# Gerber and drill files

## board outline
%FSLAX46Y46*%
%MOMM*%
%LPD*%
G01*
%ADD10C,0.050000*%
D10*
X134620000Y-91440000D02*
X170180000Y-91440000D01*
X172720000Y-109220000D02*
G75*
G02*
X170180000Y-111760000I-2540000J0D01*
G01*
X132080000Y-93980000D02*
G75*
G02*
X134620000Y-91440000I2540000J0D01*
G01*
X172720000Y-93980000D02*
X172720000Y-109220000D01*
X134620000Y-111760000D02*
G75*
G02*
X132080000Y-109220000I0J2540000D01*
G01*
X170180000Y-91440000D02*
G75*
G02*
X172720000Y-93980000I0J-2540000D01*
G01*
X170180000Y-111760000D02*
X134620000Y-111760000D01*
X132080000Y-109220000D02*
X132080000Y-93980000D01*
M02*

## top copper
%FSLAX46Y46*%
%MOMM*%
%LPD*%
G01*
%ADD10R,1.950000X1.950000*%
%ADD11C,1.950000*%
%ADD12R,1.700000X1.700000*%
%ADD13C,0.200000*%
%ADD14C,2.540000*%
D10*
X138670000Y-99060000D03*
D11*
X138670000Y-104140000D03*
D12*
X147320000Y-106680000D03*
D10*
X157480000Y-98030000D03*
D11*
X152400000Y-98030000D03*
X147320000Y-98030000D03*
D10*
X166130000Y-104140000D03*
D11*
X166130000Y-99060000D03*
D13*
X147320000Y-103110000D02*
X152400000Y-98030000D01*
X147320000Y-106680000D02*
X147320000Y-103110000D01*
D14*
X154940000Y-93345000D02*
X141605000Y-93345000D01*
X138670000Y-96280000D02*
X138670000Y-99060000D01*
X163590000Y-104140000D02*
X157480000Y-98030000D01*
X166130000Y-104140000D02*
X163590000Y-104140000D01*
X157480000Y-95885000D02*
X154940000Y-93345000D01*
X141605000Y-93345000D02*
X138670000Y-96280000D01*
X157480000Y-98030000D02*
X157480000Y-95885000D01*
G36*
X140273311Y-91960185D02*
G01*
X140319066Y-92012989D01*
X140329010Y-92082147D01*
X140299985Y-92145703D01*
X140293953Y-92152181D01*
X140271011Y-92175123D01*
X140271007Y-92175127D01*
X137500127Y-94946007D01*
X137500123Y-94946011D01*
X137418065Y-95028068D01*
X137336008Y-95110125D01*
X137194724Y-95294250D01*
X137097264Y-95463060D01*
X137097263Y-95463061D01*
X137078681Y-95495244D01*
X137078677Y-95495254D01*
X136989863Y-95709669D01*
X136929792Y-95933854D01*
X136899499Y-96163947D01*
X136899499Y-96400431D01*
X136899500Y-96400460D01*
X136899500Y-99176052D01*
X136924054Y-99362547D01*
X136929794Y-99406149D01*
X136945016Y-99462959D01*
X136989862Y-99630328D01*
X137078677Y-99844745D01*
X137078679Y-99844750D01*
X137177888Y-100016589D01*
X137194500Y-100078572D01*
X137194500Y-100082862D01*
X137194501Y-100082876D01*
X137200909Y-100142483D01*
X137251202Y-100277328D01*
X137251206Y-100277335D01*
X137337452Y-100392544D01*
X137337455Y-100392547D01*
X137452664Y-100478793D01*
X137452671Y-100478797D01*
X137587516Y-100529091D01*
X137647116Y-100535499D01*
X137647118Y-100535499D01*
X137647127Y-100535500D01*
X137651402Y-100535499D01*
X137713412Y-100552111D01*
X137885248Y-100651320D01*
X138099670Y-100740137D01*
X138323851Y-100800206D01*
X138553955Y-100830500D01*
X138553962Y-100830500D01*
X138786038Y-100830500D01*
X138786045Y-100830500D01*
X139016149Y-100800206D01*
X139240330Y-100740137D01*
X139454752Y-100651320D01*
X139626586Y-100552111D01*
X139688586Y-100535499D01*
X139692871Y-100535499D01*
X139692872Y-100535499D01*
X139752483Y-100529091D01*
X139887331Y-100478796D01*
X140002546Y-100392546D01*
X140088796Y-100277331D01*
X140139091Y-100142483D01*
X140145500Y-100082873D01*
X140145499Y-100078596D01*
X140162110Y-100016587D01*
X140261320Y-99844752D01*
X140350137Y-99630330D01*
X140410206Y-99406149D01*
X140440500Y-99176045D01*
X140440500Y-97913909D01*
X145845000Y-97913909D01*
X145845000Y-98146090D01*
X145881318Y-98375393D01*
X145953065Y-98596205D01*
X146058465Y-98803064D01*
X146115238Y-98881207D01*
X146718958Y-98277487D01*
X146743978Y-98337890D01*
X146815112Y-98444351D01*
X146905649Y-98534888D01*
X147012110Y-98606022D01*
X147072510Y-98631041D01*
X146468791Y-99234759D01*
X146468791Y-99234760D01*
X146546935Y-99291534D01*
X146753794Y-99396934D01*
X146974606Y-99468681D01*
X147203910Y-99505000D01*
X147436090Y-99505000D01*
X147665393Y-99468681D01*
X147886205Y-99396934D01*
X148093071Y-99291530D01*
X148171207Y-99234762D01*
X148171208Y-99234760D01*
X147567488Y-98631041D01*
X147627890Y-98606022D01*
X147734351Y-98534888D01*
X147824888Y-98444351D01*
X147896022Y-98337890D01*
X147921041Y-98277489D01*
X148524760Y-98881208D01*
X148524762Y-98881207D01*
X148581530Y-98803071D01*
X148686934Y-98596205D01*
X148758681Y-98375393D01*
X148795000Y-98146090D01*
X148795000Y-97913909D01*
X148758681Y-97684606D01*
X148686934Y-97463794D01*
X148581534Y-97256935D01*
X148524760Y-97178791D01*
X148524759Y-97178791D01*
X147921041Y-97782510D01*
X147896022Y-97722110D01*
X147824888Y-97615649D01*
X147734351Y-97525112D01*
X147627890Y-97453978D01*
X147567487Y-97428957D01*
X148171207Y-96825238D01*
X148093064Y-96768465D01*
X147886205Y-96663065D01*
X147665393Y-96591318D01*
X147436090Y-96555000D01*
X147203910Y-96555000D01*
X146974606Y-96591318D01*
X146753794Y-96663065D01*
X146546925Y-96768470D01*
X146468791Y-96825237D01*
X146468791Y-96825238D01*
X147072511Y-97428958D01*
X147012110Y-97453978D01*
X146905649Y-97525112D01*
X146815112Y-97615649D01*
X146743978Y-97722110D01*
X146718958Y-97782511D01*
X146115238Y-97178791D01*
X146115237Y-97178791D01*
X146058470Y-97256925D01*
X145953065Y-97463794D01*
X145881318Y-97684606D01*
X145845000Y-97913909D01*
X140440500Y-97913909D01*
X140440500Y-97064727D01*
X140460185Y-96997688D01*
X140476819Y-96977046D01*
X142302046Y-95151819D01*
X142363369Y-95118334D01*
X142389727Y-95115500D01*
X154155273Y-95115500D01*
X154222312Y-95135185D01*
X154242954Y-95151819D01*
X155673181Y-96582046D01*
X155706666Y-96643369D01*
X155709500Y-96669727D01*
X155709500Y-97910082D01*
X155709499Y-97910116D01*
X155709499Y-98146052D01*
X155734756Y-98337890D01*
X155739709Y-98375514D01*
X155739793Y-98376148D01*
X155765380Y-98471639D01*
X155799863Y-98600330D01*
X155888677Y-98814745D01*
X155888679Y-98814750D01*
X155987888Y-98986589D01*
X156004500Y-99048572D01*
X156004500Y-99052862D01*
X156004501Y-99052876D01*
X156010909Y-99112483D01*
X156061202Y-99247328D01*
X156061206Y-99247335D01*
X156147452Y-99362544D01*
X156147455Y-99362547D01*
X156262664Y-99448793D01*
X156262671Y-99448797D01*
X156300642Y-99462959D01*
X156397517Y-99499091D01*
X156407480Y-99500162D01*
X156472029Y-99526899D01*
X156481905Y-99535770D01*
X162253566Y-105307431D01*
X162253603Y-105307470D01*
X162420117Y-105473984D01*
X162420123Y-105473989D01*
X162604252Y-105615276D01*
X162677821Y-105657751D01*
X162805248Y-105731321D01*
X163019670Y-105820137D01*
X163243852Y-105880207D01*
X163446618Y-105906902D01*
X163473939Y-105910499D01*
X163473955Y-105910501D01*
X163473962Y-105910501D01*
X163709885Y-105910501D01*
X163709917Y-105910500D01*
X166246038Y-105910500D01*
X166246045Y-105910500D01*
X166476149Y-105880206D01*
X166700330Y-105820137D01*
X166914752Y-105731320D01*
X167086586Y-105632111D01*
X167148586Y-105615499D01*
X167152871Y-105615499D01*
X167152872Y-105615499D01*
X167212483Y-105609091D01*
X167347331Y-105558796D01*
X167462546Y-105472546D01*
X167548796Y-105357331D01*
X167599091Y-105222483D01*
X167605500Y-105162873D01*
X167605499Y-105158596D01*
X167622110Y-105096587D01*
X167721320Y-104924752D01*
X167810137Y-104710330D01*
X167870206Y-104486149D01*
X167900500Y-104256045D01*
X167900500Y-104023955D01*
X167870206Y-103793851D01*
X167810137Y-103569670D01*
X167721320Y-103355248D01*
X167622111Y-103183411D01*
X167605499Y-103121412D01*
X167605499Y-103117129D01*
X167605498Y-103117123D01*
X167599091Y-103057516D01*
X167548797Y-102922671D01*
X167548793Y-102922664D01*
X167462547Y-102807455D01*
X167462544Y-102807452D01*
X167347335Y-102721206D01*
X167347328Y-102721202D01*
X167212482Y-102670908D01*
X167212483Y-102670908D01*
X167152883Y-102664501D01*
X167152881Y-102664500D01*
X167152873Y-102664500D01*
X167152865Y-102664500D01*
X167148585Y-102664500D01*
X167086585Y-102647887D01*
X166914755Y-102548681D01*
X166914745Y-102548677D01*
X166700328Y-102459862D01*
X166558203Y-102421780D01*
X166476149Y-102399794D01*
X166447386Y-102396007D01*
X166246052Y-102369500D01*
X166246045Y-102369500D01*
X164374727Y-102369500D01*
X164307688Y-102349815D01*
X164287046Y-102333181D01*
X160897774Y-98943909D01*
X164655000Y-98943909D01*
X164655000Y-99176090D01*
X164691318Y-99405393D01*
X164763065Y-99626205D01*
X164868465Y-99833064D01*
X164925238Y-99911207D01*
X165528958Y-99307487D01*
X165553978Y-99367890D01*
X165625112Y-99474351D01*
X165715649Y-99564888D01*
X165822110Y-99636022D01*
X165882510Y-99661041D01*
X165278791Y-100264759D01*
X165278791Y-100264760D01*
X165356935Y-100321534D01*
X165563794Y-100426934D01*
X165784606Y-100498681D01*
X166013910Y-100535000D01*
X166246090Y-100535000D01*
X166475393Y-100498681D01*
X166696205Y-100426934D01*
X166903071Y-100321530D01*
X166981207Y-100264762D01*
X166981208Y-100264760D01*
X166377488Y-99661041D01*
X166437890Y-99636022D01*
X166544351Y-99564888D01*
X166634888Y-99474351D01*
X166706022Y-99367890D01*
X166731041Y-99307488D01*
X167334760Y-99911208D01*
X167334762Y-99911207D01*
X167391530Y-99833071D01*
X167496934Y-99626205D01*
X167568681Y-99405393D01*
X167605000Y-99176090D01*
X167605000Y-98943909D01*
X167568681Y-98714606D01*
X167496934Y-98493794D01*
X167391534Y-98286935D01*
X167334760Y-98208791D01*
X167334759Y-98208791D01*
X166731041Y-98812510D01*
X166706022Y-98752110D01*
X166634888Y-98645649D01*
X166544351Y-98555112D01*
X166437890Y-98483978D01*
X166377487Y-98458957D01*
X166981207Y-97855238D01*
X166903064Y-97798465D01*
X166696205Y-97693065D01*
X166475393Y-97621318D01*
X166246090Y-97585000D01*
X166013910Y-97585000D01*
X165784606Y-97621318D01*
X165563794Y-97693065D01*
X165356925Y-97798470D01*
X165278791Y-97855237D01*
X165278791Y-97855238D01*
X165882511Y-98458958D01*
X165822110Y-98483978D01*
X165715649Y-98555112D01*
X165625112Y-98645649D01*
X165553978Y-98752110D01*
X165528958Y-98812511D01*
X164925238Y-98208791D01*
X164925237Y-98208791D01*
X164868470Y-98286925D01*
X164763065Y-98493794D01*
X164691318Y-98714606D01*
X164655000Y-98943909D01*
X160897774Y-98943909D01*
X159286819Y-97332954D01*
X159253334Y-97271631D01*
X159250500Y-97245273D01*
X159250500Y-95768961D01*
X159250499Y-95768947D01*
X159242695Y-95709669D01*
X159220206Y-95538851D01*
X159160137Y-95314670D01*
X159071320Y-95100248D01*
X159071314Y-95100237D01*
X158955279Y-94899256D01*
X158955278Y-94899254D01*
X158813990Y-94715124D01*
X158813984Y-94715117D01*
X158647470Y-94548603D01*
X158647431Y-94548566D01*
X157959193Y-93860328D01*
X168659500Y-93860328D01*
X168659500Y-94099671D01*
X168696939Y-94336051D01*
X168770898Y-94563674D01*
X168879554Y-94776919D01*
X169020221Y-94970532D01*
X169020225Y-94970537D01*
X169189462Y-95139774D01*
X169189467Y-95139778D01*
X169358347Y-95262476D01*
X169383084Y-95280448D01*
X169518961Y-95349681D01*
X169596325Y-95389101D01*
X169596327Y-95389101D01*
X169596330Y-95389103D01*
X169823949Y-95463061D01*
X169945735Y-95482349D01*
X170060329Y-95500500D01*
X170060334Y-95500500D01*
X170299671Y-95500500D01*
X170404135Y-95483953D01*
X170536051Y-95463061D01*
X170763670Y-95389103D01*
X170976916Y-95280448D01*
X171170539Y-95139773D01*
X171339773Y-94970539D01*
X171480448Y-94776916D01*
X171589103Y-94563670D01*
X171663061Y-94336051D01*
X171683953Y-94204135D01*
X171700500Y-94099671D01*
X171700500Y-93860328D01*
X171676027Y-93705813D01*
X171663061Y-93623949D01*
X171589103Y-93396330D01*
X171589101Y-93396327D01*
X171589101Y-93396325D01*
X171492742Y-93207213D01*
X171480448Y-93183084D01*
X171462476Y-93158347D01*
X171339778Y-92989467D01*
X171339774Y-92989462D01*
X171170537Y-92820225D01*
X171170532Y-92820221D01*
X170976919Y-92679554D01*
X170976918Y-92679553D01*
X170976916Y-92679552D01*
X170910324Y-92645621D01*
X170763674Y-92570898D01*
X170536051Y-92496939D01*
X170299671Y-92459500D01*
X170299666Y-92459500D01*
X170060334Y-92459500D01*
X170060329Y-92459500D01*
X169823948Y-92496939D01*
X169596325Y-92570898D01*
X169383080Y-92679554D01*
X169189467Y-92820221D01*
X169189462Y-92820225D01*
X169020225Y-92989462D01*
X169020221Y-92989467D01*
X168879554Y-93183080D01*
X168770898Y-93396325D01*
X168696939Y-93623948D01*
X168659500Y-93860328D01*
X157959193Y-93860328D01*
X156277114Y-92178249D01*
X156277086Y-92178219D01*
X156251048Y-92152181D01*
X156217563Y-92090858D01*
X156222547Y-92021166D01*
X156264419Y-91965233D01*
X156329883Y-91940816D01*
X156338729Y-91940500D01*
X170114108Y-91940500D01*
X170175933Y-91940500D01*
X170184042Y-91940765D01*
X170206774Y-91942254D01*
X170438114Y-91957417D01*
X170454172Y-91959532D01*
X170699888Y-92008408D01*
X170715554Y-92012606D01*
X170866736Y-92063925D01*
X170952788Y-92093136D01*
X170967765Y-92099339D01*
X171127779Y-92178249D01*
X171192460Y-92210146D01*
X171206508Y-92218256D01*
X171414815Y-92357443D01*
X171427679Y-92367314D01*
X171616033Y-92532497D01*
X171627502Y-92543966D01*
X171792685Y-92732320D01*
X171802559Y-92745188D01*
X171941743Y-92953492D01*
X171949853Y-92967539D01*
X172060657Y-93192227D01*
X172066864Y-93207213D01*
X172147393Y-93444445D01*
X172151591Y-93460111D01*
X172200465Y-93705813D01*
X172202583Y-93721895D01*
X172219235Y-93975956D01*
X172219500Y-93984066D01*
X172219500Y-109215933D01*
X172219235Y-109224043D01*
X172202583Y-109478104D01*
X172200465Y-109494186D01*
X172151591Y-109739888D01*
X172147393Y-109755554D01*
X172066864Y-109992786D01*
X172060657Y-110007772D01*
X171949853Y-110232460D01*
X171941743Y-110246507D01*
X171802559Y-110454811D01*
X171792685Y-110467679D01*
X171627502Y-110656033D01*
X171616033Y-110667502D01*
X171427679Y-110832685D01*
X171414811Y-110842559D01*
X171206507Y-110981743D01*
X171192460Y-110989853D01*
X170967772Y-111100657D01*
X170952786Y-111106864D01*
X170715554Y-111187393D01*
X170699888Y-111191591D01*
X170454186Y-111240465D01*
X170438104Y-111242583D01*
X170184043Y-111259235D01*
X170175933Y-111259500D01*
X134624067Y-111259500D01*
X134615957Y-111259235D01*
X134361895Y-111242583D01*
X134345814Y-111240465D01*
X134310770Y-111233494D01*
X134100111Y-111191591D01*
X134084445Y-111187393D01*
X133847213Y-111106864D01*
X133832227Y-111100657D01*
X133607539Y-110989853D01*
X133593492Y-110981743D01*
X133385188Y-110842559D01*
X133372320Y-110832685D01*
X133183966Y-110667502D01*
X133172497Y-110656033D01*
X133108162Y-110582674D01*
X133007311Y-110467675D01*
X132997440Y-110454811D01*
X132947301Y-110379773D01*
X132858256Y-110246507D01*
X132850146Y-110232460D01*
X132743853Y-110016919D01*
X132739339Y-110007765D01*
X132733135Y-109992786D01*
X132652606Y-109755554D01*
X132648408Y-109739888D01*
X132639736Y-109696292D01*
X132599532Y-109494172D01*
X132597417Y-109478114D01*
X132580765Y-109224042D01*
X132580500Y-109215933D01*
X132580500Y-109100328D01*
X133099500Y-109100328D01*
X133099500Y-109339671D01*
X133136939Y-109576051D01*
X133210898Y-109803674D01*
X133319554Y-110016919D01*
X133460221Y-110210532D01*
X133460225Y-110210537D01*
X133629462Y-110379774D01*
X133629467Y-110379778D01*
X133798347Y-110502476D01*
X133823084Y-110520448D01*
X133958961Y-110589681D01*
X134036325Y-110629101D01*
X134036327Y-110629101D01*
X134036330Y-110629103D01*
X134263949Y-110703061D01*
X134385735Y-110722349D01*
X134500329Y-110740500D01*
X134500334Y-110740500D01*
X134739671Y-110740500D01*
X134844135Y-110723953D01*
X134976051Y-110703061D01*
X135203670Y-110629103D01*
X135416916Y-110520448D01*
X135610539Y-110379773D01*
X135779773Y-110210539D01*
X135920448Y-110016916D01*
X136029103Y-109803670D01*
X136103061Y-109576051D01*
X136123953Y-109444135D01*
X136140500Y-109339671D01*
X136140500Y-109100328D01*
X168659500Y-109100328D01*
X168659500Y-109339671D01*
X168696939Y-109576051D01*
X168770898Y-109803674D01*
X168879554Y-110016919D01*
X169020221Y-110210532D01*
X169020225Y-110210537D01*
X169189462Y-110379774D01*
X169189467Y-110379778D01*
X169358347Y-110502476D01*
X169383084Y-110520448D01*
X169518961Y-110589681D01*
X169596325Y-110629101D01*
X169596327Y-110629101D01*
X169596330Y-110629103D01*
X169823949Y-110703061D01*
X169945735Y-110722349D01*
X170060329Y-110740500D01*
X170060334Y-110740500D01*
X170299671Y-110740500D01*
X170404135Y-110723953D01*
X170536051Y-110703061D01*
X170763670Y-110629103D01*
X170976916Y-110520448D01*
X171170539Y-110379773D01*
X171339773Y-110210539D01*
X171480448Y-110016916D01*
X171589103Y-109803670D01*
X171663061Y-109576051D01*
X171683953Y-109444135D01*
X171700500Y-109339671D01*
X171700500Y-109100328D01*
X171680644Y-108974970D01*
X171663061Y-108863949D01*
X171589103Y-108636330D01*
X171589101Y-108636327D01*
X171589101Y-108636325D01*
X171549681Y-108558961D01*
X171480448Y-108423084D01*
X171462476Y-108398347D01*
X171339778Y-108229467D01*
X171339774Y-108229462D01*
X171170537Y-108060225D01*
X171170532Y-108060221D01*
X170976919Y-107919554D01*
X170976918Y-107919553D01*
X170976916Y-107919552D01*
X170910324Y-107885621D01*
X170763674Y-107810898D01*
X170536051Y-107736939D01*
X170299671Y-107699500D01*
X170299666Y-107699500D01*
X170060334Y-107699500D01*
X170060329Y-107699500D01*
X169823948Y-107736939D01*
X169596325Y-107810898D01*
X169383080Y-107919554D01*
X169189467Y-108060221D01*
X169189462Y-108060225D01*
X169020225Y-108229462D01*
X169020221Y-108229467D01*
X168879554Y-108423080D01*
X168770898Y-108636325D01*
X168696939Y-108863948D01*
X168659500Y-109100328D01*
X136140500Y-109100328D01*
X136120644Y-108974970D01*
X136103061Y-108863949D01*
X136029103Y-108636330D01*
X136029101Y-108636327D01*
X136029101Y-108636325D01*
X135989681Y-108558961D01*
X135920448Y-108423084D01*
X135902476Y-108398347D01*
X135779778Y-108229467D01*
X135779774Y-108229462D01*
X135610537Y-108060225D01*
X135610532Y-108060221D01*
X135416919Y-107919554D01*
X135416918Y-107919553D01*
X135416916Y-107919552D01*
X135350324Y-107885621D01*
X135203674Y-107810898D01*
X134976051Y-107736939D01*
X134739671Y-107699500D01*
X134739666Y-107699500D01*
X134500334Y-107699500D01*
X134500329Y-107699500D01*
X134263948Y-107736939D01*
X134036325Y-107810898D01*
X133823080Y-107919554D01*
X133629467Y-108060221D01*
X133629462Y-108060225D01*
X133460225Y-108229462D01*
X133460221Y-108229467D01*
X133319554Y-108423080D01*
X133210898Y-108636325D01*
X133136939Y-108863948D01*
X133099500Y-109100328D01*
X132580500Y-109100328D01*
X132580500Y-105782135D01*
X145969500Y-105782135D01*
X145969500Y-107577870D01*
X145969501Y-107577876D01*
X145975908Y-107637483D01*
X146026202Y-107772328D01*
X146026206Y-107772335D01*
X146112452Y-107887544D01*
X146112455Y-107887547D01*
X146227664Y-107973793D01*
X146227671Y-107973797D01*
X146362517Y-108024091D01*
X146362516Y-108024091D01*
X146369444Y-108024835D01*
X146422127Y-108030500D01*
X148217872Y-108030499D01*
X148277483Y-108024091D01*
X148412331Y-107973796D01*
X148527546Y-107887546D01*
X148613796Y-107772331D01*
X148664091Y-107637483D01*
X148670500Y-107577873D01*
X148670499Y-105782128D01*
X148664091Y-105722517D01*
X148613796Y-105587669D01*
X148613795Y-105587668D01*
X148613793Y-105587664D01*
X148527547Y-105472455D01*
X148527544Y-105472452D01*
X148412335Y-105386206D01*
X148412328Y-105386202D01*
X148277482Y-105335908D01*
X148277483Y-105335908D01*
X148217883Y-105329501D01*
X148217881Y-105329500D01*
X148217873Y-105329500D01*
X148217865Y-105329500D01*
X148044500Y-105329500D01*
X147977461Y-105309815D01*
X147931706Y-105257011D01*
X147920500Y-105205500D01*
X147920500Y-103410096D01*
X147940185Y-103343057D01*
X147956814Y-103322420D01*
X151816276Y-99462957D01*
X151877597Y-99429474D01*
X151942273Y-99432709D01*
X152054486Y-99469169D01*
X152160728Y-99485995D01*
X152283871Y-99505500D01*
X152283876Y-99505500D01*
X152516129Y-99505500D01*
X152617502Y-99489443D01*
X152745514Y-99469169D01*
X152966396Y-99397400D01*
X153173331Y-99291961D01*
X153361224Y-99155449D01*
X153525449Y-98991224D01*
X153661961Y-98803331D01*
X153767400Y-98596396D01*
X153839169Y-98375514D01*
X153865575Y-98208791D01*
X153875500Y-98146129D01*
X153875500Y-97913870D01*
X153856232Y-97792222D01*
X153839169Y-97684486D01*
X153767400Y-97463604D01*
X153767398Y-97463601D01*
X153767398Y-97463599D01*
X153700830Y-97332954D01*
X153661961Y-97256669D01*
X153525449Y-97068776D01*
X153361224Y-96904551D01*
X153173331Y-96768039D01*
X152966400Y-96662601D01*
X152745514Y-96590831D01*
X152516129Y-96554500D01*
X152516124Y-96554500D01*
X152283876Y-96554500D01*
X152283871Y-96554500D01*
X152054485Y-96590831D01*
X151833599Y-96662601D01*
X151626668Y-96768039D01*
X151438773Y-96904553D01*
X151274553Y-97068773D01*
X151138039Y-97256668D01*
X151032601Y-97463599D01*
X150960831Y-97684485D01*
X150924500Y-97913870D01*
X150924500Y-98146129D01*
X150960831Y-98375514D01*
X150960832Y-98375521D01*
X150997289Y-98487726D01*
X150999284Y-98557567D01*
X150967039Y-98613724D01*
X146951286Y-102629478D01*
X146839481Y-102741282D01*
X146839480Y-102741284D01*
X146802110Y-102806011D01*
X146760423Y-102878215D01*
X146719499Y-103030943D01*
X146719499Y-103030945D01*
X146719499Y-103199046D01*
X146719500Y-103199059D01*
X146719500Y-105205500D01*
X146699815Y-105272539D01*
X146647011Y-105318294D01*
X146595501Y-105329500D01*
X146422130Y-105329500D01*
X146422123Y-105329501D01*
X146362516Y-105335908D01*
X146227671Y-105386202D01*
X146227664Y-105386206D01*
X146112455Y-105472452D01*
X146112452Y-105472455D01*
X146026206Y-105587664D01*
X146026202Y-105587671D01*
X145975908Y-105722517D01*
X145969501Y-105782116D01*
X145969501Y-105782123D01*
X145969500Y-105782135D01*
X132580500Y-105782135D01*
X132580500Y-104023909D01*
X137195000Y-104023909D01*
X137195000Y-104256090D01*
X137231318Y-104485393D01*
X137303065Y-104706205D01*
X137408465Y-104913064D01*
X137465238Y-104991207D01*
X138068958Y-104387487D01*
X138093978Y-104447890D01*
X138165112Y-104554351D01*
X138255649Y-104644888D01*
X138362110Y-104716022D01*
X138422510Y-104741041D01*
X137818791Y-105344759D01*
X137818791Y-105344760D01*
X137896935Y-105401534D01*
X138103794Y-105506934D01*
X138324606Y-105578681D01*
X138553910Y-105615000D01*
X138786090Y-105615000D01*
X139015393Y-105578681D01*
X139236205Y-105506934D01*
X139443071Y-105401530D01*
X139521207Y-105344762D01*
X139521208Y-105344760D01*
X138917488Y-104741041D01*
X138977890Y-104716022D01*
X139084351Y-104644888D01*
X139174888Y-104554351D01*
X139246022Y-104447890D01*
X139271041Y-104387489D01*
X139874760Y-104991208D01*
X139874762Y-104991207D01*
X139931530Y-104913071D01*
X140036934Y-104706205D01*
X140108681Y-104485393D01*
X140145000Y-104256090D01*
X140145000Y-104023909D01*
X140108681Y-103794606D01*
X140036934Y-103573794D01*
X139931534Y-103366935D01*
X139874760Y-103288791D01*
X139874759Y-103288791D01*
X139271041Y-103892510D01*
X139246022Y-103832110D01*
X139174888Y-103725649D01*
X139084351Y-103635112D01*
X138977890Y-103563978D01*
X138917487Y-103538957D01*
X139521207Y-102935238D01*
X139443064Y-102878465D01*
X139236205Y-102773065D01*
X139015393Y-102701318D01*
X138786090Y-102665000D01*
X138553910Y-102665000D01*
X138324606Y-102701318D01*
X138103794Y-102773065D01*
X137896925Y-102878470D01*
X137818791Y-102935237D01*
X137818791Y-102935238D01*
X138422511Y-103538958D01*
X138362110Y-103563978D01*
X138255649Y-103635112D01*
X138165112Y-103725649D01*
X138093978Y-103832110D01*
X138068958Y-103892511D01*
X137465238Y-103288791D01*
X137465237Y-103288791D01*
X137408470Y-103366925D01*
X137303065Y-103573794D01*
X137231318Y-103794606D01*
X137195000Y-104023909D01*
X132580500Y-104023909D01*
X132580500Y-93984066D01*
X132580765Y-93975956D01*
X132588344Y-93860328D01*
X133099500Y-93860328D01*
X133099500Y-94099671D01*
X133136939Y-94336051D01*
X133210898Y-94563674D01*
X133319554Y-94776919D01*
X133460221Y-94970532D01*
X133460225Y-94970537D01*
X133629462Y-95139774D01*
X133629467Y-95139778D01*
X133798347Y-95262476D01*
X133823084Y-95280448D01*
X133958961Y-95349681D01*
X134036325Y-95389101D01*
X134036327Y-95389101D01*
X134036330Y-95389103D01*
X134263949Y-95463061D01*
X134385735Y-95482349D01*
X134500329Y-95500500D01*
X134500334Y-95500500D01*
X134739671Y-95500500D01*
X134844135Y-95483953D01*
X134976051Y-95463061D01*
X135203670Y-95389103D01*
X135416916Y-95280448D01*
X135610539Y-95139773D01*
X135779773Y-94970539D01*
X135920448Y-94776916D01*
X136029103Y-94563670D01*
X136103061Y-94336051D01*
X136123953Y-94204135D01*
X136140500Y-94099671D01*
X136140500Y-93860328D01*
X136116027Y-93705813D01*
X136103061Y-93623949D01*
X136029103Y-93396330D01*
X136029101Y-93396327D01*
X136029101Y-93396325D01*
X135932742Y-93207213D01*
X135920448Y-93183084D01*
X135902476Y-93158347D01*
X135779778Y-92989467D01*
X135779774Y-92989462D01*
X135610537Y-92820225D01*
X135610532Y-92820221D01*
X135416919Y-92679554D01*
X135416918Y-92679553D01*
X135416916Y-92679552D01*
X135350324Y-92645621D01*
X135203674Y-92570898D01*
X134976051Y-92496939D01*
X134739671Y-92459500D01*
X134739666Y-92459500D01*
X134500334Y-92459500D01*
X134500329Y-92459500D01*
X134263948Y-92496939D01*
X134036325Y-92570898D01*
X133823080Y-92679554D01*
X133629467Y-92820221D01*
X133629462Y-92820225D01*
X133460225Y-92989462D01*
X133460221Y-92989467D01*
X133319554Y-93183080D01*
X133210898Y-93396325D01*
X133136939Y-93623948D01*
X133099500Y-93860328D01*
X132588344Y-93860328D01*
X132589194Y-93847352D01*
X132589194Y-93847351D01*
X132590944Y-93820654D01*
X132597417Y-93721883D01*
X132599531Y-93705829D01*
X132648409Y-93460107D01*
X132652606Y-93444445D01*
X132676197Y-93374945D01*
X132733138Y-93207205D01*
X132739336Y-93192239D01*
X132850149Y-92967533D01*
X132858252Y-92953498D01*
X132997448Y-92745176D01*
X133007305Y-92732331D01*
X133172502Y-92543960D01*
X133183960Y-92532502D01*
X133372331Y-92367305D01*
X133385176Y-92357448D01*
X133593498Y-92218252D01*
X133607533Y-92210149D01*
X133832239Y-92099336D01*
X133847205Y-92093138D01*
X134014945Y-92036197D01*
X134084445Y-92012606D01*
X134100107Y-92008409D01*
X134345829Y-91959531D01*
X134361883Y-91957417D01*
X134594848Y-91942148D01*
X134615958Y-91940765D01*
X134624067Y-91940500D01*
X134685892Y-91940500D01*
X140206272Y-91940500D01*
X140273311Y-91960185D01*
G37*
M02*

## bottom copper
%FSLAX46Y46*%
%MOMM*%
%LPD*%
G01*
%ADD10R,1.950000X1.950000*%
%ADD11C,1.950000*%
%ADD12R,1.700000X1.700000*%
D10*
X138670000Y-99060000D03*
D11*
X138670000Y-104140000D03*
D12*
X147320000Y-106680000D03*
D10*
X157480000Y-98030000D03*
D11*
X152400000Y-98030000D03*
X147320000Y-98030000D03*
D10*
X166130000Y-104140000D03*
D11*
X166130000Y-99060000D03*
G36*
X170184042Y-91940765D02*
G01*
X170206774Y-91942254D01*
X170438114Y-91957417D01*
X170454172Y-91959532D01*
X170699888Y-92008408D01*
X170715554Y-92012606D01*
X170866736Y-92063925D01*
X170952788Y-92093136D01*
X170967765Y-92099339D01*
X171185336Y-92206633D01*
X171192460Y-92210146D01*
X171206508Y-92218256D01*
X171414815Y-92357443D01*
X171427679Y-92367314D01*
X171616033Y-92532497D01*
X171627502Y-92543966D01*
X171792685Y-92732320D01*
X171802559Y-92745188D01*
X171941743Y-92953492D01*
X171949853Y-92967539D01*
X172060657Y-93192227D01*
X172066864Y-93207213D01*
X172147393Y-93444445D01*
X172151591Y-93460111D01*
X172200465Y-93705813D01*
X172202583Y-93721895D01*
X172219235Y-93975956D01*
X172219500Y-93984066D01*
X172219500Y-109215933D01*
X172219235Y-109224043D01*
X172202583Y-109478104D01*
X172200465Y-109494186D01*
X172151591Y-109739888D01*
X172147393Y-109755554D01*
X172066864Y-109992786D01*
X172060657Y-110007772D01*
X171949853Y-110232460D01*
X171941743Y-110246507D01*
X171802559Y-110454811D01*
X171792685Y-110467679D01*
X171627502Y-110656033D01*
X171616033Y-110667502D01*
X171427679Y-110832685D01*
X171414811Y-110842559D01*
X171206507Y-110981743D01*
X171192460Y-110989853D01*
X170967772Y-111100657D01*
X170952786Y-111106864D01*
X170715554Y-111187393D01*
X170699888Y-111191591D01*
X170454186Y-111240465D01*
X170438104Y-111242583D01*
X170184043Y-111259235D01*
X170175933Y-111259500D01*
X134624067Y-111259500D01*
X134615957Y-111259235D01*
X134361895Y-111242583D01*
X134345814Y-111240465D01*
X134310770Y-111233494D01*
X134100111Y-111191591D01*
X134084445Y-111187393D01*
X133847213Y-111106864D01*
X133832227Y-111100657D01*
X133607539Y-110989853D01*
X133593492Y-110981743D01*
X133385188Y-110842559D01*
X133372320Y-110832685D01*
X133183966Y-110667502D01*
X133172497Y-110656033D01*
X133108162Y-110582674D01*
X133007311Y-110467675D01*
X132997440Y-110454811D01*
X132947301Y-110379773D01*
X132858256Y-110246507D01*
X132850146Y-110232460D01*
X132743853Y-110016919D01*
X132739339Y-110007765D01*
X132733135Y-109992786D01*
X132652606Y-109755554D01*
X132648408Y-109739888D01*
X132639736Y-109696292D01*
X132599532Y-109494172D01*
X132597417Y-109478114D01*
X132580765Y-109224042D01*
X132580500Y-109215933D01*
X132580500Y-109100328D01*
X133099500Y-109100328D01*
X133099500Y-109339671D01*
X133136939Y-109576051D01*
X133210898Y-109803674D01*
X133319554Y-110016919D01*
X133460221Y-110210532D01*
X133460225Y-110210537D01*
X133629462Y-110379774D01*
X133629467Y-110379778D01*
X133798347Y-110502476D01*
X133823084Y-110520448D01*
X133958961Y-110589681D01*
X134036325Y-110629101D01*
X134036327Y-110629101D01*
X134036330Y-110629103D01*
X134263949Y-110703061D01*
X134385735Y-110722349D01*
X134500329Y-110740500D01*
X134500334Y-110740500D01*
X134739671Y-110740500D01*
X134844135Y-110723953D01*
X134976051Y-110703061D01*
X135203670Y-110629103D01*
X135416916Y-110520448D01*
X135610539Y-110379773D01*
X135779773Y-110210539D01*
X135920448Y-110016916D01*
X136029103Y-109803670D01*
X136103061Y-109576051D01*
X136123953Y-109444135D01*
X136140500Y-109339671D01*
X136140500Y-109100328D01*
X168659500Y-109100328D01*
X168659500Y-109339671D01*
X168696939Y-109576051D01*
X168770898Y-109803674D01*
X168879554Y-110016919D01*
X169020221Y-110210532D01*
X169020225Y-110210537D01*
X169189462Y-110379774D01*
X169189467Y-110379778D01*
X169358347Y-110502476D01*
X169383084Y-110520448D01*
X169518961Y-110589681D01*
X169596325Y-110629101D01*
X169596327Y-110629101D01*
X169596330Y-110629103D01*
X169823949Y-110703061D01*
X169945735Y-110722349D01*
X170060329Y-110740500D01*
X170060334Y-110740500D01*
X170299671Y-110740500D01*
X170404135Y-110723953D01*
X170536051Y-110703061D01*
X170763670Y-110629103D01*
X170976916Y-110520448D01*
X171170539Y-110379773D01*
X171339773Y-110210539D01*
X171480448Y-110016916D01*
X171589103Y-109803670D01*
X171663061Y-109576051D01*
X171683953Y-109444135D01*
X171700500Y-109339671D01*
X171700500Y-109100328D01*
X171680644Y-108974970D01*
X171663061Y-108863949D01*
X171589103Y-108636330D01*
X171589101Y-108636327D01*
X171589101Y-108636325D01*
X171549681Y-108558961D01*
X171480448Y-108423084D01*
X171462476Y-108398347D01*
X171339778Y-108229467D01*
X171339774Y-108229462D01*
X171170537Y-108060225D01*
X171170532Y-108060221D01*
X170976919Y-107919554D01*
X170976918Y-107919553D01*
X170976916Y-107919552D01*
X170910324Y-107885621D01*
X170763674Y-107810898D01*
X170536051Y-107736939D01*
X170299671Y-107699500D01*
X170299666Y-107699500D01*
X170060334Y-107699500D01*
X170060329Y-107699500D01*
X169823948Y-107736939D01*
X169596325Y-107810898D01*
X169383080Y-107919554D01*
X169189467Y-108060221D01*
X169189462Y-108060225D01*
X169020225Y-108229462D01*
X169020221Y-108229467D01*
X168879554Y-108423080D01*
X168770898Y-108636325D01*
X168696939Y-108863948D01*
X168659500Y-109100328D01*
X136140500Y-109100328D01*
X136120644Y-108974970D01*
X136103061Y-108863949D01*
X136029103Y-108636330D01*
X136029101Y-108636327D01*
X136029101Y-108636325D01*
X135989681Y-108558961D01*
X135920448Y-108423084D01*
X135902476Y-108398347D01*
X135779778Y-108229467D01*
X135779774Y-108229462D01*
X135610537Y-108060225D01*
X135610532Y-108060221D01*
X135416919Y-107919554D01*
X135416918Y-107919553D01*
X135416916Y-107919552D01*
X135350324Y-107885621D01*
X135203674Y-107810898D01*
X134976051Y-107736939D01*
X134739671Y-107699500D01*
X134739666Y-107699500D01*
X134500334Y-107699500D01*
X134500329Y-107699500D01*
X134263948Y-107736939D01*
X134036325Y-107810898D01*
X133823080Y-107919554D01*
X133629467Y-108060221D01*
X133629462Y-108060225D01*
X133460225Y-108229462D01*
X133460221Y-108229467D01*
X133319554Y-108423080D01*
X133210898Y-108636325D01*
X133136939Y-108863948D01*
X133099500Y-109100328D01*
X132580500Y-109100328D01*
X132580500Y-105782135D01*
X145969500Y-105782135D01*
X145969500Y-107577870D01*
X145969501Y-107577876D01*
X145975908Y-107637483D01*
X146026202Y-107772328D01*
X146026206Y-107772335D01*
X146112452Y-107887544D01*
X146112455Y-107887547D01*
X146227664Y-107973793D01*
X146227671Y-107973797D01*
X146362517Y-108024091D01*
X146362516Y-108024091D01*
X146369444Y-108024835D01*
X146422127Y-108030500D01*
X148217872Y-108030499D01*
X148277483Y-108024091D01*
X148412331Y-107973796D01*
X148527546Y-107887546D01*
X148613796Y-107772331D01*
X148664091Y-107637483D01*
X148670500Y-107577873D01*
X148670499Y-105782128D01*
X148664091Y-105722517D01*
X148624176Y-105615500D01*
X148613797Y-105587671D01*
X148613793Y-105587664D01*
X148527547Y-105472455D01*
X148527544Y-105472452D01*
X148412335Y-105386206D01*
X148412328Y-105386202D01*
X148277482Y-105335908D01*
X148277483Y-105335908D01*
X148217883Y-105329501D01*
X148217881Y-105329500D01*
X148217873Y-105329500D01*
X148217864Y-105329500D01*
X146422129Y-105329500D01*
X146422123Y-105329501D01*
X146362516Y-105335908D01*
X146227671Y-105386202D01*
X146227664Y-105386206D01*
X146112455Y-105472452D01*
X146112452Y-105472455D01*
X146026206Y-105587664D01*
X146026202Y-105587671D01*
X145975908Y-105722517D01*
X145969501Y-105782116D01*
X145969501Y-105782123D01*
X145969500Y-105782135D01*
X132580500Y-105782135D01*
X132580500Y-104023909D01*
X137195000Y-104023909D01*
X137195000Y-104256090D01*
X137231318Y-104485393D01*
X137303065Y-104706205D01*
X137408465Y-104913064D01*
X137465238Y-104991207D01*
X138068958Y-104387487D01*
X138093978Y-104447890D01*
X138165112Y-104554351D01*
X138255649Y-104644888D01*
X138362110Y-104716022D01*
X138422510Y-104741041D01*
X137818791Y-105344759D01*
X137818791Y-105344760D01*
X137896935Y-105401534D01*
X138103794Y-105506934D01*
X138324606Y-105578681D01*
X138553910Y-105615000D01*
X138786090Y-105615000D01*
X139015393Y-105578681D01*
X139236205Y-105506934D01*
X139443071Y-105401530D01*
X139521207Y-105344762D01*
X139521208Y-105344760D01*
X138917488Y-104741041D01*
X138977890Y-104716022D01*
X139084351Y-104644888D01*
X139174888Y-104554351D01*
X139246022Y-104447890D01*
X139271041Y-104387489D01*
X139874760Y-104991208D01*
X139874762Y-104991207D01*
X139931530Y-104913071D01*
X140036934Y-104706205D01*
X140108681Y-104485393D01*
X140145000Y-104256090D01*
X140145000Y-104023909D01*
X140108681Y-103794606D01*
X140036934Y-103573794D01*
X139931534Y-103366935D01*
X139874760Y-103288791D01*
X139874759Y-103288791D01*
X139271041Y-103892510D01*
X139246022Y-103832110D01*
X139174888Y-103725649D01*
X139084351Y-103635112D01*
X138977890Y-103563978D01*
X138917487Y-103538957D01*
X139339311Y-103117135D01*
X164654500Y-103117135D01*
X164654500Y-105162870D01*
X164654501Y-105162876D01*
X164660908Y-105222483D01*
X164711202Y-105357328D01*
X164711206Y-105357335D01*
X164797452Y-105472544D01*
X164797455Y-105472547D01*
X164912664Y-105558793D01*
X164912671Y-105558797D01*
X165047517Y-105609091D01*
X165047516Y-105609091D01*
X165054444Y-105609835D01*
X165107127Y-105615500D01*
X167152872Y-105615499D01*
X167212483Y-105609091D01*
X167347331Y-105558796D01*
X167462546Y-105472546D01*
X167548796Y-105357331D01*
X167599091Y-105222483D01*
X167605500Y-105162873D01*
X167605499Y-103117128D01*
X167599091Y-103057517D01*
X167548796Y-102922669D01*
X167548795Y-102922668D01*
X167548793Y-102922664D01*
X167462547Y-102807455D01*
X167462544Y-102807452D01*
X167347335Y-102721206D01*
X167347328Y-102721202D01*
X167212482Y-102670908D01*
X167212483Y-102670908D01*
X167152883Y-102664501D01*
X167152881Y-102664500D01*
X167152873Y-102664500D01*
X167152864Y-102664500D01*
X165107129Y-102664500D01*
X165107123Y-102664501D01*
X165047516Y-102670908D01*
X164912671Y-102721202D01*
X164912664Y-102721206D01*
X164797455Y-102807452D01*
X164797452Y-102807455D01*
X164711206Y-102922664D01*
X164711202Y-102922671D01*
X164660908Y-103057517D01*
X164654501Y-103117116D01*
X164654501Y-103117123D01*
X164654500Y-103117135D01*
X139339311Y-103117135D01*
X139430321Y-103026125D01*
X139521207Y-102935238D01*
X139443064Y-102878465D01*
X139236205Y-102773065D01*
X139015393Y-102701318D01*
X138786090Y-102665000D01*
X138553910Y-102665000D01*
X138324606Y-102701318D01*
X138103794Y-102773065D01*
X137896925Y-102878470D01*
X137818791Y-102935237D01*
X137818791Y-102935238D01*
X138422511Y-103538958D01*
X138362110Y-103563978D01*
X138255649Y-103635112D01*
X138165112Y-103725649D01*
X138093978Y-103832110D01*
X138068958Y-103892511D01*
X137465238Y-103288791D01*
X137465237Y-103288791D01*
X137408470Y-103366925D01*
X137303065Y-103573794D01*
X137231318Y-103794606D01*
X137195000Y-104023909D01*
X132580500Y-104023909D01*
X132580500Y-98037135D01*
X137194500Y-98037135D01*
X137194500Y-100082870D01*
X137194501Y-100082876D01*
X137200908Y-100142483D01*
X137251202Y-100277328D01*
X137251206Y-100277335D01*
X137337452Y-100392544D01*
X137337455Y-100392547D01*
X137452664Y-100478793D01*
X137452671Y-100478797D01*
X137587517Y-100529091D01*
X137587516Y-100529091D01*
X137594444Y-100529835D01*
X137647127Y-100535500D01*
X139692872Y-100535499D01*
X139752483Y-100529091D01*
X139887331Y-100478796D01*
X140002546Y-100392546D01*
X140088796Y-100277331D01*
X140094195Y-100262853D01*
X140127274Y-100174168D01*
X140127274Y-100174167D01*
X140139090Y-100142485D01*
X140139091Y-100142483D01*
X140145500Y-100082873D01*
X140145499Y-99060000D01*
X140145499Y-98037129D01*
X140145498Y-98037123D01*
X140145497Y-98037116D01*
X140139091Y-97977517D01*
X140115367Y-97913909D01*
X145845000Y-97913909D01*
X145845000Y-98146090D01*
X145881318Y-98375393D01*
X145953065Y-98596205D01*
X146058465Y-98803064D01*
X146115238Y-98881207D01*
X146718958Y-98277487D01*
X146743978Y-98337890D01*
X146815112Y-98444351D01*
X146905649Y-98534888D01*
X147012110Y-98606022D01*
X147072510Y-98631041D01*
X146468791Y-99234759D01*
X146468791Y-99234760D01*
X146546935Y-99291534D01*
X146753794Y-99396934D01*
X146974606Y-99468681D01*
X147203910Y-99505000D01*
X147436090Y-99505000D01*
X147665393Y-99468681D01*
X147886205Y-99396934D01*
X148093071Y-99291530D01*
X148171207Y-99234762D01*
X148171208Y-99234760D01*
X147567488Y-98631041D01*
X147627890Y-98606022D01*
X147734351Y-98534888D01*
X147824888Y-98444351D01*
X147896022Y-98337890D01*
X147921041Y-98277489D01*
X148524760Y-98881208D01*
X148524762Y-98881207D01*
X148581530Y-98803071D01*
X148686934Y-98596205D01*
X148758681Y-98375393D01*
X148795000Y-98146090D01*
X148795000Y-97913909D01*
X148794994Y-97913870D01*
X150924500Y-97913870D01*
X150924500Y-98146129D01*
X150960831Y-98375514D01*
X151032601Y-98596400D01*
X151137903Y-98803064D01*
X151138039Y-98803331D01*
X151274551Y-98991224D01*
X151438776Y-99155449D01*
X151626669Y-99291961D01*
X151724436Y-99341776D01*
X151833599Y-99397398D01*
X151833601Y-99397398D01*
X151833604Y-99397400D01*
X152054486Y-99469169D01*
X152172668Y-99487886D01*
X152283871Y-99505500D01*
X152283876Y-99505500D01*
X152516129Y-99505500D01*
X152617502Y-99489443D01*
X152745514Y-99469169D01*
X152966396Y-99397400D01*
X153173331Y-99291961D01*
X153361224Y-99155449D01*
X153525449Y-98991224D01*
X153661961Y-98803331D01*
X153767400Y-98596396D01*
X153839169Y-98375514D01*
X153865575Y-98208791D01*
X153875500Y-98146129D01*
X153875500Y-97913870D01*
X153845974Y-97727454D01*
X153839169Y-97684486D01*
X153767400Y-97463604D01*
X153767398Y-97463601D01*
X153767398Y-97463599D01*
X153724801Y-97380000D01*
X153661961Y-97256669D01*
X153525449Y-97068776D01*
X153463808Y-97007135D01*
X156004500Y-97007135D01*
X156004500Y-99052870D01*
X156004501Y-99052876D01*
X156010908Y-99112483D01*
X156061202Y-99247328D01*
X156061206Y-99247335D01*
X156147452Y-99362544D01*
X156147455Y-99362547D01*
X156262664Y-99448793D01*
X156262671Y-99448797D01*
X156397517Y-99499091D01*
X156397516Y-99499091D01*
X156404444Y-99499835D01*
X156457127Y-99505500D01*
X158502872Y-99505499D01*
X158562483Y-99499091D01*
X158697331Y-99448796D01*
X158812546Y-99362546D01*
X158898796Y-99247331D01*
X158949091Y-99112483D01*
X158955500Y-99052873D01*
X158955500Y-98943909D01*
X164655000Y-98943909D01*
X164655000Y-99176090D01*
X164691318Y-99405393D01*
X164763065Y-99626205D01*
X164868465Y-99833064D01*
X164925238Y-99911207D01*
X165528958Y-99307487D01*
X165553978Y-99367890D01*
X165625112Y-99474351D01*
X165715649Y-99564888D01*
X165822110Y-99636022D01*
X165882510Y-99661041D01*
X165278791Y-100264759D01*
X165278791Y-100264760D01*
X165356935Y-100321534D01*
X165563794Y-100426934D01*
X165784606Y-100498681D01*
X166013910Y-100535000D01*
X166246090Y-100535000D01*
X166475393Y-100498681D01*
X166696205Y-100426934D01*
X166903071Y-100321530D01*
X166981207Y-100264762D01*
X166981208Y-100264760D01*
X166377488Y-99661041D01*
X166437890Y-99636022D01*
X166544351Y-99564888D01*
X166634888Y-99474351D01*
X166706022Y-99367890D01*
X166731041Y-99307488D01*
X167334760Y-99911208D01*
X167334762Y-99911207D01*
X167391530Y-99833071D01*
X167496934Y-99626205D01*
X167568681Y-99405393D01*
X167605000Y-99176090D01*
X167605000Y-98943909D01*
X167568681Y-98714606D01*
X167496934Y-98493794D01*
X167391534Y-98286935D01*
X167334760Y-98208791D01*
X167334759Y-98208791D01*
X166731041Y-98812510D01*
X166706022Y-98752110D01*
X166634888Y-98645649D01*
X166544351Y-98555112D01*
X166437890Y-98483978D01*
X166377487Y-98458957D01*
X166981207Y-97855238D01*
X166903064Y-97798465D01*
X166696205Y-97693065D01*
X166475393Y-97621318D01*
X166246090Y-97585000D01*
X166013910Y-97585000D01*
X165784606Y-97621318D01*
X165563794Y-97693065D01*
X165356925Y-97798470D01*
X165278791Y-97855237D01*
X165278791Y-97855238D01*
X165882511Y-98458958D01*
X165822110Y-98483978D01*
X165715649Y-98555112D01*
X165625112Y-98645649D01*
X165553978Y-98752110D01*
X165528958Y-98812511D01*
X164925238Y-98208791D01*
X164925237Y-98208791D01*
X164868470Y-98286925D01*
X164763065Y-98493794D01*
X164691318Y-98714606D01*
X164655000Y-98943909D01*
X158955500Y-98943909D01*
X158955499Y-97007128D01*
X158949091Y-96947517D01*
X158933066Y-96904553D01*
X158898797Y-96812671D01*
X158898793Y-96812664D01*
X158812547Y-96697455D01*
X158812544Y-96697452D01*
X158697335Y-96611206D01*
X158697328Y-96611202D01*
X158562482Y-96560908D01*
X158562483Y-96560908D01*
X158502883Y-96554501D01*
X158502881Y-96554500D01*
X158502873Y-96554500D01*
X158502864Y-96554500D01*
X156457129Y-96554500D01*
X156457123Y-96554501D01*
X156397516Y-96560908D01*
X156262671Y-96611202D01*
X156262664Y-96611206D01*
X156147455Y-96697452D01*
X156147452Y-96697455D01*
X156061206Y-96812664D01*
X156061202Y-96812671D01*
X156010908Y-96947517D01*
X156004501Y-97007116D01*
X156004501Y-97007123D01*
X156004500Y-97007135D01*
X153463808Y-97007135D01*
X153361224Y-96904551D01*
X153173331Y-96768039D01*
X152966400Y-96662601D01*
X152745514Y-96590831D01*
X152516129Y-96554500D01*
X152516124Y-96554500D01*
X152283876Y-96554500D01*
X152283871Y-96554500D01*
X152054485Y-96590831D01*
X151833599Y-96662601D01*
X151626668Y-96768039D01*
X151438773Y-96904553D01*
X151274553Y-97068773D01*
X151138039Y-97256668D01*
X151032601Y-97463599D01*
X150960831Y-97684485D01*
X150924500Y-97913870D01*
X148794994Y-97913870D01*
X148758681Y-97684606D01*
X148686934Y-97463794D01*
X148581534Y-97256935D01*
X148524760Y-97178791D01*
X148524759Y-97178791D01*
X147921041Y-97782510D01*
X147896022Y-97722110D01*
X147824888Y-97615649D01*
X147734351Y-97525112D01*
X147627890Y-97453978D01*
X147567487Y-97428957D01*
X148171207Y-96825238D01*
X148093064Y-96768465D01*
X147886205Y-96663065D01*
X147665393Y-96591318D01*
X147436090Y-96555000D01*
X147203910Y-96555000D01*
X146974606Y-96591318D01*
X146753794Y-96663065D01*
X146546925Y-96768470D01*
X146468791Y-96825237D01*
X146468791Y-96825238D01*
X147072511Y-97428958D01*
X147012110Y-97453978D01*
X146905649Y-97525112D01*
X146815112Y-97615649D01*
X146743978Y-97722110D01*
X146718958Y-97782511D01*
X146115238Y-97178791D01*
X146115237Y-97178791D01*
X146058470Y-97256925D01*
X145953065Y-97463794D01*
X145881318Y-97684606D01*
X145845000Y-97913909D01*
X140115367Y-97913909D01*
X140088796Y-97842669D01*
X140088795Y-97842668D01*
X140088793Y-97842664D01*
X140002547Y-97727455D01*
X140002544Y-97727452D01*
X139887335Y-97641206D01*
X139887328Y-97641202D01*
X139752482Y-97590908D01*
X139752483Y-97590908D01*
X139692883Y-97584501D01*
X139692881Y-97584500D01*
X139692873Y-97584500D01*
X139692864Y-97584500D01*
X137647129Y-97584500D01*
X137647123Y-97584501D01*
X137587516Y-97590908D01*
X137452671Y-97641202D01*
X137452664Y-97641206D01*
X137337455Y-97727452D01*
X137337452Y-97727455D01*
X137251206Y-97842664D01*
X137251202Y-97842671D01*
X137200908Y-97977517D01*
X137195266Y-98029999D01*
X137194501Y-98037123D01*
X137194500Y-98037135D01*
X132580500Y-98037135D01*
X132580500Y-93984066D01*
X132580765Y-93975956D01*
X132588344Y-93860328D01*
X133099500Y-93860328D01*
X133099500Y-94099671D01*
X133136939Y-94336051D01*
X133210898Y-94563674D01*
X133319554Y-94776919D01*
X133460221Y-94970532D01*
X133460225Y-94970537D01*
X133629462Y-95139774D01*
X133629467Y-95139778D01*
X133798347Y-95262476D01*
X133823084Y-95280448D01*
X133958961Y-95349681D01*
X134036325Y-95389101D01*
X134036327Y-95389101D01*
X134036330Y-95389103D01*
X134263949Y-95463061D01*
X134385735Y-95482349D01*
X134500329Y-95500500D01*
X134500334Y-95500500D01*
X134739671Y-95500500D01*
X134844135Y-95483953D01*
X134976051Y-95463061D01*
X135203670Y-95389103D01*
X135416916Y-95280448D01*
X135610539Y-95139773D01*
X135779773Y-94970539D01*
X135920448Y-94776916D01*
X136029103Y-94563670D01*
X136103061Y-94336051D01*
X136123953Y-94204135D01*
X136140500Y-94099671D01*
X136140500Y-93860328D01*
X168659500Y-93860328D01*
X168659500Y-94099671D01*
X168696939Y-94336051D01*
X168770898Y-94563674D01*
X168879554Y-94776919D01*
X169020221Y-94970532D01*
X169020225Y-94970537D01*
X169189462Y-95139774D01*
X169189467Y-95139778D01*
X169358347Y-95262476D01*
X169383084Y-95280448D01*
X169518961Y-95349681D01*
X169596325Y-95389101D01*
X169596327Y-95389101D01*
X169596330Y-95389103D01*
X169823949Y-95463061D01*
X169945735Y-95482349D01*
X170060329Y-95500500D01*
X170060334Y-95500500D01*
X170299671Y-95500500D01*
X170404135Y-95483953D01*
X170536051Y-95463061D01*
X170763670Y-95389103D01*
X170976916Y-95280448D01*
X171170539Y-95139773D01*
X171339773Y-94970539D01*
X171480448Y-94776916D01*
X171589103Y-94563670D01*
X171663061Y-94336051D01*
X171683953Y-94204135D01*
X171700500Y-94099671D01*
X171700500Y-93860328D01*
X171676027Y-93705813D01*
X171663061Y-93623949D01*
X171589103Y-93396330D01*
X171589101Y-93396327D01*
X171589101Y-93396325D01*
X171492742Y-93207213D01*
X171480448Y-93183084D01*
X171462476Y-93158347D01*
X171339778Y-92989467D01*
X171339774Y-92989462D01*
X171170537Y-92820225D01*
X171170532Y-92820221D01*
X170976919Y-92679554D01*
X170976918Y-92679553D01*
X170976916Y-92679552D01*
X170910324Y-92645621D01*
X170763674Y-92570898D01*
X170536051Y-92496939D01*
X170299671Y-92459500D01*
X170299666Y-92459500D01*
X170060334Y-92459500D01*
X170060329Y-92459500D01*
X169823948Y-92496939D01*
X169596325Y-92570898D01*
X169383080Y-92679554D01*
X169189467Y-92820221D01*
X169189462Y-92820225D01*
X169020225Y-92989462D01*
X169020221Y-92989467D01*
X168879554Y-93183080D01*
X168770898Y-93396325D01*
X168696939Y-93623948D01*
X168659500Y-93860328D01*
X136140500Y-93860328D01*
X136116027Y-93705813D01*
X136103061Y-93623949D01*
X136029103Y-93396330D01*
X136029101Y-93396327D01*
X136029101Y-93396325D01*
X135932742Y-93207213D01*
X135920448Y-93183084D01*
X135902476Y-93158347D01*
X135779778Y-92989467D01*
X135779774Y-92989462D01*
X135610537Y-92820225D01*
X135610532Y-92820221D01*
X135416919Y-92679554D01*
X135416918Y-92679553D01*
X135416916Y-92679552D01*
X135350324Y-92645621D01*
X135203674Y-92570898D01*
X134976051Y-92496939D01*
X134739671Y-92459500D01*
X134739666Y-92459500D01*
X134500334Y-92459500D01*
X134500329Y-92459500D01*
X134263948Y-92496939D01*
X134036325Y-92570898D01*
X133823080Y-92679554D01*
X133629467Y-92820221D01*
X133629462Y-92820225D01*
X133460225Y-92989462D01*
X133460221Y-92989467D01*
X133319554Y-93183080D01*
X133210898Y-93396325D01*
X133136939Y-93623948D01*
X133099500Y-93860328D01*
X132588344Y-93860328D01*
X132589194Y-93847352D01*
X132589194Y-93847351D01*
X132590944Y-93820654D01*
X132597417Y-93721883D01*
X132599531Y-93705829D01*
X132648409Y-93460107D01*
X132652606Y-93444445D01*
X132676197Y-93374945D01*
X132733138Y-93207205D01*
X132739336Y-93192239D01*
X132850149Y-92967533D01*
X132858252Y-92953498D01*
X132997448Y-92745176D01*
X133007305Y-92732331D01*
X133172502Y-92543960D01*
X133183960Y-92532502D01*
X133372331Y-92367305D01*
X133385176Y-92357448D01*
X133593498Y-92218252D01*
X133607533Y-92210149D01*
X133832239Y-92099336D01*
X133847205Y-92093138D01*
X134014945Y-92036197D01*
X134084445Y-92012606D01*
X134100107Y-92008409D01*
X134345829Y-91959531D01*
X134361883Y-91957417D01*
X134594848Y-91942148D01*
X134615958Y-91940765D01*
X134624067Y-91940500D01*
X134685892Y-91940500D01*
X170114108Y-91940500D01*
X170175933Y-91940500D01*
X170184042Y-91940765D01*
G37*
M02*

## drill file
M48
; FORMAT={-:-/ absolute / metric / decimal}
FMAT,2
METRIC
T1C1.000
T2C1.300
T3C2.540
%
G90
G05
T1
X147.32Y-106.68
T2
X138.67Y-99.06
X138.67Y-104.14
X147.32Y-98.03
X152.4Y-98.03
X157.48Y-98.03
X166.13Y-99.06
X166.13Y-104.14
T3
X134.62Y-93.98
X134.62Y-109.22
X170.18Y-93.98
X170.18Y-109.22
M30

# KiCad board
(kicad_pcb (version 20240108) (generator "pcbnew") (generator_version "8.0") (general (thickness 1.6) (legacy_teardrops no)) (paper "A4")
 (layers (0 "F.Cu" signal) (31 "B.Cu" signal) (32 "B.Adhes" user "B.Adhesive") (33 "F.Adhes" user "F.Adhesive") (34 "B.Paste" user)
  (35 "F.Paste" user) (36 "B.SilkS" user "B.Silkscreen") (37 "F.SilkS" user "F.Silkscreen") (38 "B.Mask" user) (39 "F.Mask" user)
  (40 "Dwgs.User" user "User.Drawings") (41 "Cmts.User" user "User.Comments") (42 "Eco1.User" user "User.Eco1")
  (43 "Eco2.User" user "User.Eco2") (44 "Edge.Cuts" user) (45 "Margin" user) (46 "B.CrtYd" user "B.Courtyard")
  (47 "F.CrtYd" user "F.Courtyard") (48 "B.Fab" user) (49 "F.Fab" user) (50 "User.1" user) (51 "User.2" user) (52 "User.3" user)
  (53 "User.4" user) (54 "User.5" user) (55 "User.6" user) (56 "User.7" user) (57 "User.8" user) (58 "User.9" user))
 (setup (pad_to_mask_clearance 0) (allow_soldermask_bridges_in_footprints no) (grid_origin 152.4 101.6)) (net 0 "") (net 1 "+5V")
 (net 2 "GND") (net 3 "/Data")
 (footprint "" (layer "F.Cu") (at 134.62 109.22)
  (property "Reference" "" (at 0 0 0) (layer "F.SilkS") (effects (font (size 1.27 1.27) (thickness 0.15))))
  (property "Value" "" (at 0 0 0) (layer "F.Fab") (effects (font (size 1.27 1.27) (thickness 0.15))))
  (pad "" np_thru_hole circle (at 0 0) (size 2.5 2.5) (drill 2.54) (layers "F&B.Cu" "*.Mask")))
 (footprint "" (layer "F.Cu") (at 170.18 93.98)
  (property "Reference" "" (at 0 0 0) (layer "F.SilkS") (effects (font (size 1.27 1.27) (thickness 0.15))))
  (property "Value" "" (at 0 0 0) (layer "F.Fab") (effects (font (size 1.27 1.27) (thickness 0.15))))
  (pad "" np_thru_hole circle (at 0 0) (size 2.5 2.5) (drill 2.54) (layers "F&B.Cu" "*.Mask")))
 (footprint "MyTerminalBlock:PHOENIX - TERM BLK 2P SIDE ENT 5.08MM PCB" (layer "F.Cu") (at 134.62 96.52 -90)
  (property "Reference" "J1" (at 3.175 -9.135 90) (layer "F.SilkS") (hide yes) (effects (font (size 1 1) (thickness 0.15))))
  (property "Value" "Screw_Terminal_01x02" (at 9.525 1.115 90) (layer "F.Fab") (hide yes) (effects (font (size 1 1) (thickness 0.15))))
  (pad "1" thru_hole rect (at 2.54 -4.05 270) (size 1.95 1.95) (drill 1.3) (layers "*.Cu" "*.Mask") (remove_unused_layers no) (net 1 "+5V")
   (solder_mask_margin 0.102))
  (pad "2" thru_hole circle (at 7.62 -4.05 270) (size 1.95 1.95) (drill 1.3) (layers "*.Cu" "*.Mask") (remove_unused_layers no)
   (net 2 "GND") (solder_mask_margin 0.102)))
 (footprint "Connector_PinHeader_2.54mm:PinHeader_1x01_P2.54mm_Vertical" (layer "F.Cu") (at 147.32 106.68 -90)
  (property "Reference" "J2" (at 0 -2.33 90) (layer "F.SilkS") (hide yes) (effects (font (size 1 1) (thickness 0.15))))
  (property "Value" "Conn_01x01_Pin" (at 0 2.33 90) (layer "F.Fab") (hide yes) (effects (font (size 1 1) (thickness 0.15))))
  (pad "1" thru_hole rect (at 0 0 270) (size 1.7 1.7) (drill 1) (layers "*.Cu" "*.Mask") (remove_unused_layers no) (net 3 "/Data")))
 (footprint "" (layer "F.Cu") (at 134.62 93.98)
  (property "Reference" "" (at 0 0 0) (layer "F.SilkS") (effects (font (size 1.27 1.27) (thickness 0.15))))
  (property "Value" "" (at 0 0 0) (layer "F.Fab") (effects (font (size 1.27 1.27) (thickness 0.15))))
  (pad "" np_thru_hole circle (at 0 0) (size 2.5 2.5) (drill 2.54) (layers "F&B.Cu" "*.Mask")))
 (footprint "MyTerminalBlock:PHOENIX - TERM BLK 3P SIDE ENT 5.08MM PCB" (layer "F.Cu") (at 160.02 93.98 180)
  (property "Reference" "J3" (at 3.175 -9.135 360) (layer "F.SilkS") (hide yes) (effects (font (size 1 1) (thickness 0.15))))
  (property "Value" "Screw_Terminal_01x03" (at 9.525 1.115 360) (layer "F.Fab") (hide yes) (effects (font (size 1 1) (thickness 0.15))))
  (pad "1" thru_hole rect (at 2.54 -4.05 180) (size 1.95 1.95) (drill 1.3) (layers "*.Cu" "*.Mask") (remove_unused_layers no) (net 1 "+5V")
   (solder_mask_margin 0.102))
  (pad "2" thru_hole circle (at 7.62 -4.05 180) (size 1.95 1.95) (drill 1.3) (layers "*.Cu" "*.Mask") (remove_unused_layers no)
   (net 3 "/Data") (solder_mask_margin 0.102))
  (pad "3" thru_hole circle (at 12.7 -4.05 180) (size 1.95 1.95) (drill 1.3) (layers "*.Cu" "*.Mask") (remove_unused_layers no)
   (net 2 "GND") (solder_mask_margin 0.102)))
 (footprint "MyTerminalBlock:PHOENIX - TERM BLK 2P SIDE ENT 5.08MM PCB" (layer "F.Cu") (at 170.18 106.68 90)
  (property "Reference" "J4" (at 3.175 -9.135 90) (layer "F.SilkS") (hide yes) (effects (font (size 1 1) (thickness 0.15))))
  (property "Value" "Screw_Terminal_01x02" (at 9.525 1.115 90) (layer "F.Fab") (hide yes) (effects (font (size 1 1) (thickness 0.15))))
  (pad "1" thru_hole rect (at 2.54 -4.05 90) (size 1.95 1.95) (drill 1.3) (layers "*.Cu" "*.Mask") (remove_unused_layers no) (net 1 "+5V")
   (solder_mask_margin 0.102))
  (pad "2" thru_hole circle (at 7.62 -4.05 90) (size 1.95 1.95) (drill 1.3) (layers "*.Cu" "*.Mask") (remove_unused_layers no) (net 2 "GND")
   (solder_mask_margin 0.102)))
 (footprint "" (layer "F.Cu") (at 170.18 109.22)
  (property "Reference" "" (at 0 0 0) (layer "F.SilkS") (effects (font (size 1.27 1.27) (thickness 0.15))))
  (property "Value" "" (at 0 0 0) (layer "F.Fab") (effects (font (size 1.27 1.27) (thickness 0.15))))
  (pad "" np_thru_hole circle (at 0 0) (size 2.5 2.5) (drill 2.54) (layers "F&B.Cu" "*.Mask")))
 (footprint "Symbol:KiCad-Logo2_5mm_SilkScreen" (layer "B.Cu") (at 156.845 106.045 180)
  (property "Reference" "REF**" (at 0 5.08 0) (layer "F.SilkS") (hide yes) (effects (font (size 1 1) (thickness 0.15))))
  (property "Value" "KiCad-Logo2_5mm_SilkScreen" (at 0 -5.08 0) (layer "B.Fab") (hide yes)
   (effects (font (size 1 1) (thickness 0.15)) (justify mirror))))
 (gr_line (start 134.62 91.44) (end 170.18 91.44) (stroke (width 0.05) (type default)) (layer "Edge.Cuts"))
 (gr_arc (start 172.72 109.22) (mid 171.976051 111.016051) (end 170.18 111.76) (stroke (width 0.05) (type default)) (layer "Edge.Cuts"))
 (gr_arc (start 132.08 93.98) (mid 132.823949 92.183949) (end 134.62 91.44) (stroke (width 0.05) (type default)) (layer "Edge.Cuts"))
 (gr_line (start 172.72 93.98) (end 172.72 109.22) (stroke (width 0.05) (type default)) (layer "Edge.Cuts"))
 (gr_arc (start 134.62 111.76) (mid 132.823949 111.016051) (end 132.08 109.22) (stroke (width 0.05) (type default)) (layer "Edge.Cuts"))
 (gr_arc (start 170.18 91.44) (mid 171.976051 92.183949) (end 172.72 93.98) (stroke (width 0.05) (type default)) (layer "Edge.Cuts"))
 (gr_line (start 170.18 111.76) (end 134.62 111.76) (stroke (width 0.05) (type default)) (layer "Edge.Cuts"))
 (gr_line (start 132.08 109.22) (end 132.08 93.98) (stroke (width 0.05) (type default)) (layer "Edge.Cuts"))
 (segment (start 147.32 103.11) (end 152.4 98.03) (width 0.2) (layer "F.Cu") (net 3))
 (segment (start 147.32 106.68) (end 147.32 103.11) (width 0.2) (layer "F.Cu") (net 3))
 (segment (start 154.94 93.345) (end 141.605 93.345) (width 2.54) (layer "F.Cu") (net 1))
 (segment (start 138.67 96.28) (end 138.67 99.06) (width 2.54) (layer "F.Cu") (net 1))
 (segment (start 163.59 104.14) (end 157.48 98.03) (width 2.54) (layer "F.Cu") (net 1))
 (segment (start 166.13 104.14) (end 163.59 104.14) (width 2.54) (layer "F.Cu") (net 1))
 (segment (start 157.48 95.885) (end 154.94 93.345) (width 2.54) (layer "F.Cu") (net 1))
 (segment (start 141.605 93.345) (end 138.67 96.28) (width 2.54) (layer "F.Cu") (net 1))
 (segment (start 157.48 98.03) (end 157.48 95.885) (width 2.54) (layer "F.Cu") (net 1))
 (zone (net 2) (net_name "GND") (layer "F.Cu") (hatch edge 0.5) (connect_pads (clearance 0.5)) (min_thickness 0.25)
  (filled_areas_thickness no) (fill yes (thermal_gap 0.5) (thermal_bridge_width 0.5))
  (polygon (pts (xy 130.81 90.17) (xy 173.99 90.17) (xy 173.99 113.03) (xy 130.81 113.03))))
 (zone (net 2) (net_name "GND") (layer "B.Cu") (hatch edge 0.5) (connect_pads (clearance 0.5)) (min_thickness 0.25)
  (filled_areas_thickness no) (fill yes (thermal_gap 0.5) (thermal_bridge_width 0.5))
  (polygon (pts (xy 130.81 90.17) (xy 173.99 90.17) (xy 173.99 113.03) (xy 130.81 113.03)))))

